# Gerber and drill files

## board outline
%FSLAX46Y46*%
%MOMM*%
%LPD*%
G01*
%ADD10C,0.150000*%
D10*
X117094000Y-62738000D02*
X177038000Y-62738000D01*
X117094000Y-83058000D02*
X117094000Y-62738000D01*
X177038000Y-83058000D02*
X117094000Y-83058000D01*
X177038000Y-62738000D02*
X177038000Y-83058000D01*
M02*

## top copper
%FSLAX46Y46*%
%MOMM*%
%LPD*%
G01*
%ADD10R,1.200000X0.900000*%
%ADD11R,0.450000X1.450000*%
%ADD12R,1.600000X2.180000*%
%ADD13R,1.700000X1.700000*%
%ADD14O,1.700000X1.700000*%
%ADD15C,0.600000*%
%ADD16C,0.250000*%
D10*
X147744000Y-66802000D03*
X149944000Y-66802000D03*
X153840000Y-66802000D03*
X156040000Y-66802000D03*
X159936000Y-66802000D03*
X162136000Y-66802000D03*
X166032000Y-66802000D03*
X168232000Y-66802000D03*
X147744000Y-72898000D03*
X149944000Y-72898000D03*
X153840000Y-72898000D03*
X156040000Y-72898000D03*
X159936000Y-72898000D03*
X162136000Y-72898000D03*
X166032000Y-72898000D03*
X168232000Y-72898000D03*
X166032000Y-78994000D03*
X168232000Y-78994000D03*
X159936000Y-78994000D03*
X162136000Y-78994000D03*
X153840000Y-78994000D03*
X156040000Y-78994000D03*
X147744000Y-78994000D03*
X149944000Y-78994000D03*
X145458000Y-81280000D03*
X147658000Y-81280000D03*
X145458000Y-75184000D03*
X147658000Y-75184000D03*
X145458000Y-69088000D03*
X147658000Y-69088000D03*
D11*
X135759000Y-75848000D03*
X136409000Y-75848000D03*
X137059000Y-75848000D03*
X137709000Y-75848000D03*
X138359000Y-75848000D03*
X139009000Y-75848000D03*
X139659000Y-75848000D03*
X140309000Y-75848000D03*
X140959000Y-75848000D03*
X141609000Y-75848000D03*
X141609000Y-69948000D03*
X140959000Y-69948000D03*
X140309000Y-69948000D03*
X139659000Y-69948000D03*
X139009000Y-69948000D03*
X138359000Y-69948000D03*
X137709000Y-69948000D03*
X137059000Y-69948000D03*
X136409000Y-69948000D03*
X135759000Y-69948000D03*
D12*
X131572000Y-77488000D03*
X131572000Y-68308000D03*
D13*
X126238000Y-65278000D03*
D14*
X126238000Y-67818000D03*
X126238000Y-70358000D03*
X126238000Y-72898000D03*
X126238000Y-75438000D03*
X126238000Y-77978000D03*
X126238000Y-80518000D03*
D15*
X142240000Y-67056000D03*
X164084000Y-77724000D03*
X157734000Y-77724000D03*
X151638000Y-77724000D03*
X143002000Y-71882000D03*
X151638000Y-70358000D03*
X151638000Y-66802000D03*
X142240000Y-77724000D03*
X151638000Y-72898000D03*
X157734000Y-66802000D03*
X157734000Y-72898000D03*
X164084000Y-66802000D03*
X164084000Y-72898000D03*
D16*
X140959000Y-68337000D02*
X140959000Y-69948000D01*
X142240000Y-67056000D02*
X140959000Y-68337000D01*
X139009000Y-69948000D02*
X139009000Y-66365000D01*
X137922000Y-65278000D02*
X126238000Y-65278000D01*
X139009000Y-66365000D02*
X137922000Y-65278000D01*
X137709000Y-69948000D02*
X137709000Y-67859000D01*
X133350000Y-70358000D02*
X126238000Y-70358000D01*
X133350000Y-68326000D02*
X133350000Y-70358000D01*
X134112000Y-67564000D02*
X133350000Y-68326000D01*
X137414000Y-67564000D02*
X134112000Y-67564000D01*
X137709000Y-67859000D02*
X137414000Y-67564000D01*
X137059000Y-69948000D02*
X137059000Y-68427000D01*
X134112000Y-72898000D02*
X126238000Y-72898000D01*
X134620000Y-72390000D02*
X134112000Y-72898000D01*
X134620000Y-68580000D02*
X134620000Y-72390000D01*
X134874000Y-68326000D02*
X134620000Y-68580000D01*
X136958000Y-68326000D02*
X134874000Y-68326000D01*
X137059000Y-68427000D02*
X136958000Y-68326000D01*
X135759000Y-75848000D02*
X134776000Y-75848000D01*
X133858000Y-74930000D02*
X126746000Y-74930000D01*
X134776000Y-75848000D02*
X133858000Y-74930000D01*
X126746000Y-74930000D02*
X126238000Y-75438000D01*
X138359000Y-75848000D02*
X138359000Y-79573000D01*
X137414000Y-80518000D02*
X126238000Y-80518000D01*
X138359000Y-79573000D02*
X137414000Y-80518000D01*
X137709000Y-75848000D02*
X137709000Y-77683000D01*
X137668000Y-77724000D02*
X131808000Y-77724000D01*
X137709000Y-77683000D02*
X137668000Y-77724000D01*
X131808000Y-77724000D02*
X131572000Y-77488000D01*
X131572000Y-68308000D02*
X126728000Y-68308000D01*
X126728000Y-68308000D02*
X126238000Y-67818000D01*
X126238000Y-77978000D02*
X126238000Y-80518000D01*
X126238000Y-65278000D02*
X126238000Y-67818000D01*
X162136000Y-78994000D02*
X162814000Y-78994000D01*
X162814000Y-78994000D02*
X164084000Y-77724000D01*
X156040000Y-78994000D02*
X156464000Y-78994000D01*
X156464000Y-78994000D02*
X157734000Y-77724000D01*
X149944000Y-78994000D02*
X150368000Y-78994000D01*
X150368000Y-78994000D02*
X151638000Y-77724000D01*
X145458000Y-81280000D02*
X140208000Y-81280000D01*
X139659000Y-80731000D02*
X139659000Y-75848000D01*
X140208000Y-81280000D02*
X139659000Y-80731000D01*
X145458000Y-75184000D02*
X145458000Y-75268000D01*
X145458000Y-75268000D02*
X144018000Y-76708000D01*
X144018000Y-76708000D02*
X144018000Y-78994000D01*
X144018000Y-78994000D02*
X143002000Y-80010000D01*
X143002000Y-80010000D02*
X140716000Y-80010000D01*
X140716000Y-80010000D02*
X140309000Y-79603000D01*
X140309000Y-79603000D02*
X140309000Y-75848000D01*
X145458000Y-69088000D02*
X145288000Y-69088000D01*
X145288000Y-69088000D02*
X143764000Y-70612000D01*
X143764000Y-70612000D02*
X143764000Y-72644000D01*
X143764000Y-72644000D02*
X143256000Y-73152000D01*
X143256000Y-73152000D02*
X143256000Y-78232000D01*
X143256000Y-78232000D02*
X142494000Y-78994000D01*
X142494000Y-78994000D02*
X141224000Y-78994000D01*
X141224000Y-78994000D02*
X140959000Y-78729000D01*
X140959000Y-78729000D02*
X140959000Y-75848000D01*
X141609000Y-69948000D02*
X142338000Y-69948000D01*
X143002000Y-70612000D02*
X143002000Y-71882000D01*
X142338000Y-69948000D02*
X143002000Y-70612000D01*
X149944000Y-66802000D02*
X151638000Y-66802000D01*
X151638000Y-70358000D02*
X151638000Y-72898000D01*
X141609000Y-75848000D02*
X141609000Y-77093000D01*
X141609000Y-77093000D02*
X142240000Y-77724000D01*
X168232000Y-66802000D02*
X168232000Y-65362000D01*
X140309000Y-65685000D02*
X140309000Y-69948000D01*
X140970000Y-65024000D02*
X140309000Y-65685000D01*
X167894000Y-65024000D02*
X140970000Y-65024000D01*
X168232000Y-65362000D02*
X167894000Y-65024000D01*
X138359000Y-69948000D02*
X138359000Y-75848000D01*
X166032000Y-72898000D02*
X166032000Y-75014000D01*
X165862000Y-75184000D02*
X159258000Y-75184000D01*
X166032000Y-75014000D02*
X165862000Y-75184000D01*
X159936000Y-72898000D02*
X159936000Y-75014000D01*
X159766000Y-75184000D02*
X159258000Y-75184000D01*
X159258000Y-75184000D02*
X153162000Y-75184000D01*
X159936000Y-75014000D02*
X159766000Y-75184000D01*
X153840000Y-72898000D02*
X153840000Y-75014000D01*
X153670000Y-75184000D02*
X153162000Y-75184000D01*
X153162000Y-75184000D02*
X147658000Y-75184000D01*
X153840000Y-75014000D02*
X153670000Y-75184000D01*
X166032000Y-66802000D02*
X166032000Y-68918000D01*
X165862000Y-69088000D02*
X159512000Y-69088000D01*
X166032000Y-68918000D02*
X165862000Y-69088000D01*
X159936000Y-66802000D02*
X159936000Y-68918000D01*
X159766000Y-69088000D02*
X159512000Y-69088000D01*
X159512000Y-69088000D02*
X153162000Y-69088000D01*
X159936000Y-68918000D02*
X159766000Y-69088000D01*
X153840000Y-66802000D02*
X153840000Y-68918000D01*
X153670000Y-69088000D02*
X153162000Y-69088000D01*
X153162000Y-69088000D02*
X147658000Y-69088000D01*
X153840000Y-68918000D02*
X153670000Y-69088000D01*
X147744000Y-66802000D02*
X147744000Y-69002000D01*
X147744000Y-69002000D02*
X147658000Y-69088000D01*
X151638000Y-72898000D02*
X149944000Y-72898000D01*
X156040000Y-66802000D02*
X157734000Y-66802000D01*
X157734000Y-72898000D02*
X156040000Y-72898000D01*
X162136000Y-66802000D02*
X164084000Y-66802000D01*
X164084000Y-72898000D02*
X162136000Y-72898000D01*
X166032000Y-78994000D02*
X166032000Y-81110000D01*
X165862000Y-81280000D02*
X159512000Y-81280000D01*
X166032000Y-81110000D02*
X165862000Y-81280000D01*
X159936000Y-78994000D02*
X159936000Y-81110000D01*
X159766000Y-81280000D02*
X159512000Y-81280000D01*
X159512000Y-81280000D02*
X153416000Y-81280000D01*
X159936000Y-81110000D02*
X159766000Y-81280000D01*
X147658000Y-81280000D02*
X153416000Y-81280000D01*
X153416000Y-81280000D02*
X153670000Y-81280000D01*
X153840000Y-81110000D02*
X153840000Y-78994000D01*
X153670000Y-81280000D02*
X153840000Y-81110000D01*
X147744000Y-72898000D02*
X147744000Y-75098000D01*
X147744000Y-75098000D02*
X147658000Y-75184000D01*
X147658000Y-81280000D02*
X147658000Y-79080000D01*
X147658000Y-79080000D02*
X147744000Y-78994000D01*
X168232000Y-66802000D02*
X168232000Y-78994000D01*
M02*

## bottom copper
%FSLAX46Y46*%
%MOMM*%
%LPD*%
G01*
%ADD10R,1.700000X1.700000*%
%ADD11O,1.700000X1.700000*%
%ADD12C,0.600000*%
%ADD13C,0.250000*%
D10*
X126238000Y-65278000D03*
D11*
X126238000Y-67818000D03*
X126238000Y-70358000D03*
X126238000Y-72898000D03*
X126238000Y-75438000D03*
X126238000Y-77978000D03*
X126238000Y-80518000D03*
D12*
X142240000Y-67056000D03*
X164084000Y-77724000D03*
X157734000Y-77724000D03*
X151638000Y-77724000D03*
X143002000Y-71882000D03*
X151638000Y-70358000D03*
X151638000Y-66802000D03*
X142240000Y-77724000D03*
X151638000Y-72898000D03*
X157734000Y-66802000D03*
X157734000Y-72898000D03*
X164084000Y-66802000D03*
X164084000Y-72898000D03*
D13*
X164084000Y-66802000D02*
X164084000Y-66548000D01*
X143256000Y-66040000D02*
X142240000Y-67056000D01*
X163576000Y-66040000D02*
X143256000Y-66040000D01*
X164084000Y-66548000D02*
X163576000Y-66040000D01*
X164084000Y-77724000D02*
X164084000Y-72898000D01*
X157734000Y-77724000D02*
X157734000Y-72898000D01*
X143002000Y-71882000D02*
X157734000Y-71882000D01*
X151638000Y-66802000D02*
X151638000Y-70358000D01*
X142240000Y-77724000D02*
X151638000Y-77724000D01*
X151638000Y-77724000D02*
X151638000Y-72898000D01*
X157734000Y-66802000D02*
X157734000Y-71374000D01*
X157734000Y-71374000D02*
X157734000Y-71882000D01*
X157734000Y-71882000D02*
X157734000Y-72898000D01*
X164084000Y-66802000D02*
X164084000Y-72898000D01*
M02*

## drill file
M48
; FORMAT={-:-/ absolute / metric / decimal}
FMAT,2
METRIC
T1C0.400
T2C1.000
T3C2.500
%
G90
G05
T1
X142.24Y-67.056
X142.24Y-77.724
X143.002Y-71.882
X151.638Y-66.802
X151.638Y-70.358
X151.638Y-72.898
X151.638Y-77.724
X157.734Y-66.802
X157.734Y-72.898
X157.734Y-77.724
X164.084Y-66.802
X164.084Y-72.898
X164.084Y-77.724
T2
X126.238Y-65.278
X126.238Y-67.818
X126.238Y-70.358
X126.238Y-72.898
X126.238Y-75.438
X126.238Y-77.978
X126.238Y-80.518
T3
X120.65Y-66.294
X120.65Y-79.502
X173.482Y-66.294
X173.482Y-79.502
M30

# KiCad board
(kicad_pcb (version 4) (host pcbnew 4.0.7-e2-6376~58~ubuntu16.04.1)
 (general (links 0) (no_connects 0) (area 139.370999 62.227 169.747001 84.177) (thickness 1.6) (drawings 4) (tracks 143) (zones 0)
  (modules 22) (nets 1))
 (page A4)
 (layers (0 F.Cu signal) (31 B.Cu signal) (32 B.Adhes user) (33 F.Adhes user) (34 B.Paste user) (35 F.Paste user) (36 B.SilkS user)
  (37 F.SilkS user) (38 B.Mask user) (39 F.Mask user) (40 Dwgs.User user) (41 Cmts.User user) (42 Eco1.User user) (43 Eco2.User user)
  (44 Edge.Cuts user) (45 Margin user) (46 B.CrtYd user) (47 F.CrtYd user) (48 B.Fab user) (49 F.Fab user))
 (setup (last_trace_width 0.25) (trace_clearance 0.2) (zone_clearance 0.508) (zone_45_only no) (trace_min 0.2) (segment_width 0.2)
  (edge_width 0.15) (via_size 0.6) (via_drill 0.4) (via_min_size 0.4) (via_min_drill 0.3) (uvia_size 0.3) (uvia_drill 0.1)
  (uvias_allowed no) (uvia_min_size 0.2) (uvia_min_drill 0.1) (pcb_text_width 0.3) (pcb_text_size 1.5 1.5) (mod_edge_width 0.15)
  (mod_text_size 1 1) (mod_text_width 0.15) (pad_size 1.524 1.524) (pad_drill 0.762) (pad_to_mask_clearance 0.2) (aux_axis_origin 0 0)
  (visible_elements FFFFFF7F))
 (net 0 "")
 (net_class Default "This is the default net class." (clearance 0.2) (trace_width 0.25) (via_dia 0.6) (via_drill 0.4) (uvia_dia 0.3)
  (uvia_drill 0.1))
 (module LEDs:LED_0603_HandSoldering (layer F.Cu) (at 148.844 66.802)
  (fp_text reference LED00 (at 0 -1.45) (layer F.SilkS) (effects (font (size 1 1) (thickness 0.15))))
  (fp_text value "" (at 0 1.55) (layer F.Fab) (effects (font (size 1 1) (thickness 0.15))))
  (pad 1 smd rect (at -1.1 0) (size 1.2 0.9) (layers F.Cu F.Paste F.Mask))
  (pad 2 smd rect (at 1.1 0) (size 1.2 0.9) (layers F.Cu F.Paste F.Mask)))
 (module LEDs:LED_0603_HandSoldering (layer F.Cu) (at 154.94 66.802)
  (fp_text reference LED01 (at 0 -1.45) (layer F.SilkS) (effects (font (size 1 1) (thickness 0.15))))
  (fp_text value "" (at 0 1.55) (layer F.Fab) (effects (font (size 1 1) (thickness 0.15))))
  (pad 1 smd rect (at -1.1 0) (size 1.2 0.9) (layers F.Cu F.Paste F.Mask))
  (pad 2 smd rect (at 1.1 0) (size 1.2 0.9) (layers F.Cu F.Paste F.Mask)))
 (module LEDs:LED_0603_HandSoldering (layer F.Cu) (at 161.036 66.802)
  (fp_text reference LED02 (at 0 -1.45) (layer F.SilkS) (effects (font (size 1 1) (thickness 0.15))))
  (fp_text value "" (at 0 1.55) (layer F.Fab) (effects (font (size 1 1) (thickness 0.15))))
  (pad 1 smd rect (at -1.1 0) (size 1.2 0.9) (layers F.Cu F.Paste F.Mask))
  (pad 2 smd rect (at 1.1 0) (size 1.2 0.9) (layers F.Cu F.Paste F.Mask)))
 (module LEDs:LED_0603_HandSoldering (layer F.Cu) (at 167.132 66.802)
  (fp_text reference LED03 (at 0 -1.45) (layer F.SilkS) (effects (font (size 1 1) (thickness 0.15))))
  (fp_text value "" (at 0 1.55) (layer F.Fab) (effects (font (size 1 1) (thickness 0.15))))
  (pad 1 smd rect (at -1.1 0) (size 1.2 0.9) (layers F.Cu F.Paste F.Mask))
  (pad 2 smd rect (at 1.1 0) (size 1.2 0.9) (layers F.Cu F.Paste F.Mask)))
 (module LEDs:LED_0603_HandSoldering (layer F.Cu) (at 148.844 72.898)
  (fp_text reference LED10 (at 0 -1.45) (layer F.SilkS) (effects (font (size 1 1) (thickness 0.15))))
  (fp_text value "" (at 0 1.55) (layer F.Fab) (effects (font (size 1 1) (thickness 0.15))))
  (pad 1 smd rect (at -1.1 0) (size 1.2 0.9) (layers F.Cu F.Paste F.Mask))
  (pad 2 smd rect (at 1.1 0) (size 1.2 0.9) (layers F.Cu F.Paste F.Mask)))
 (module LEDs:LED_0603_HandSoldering (layer F.Cu) (at 154.94 72.898)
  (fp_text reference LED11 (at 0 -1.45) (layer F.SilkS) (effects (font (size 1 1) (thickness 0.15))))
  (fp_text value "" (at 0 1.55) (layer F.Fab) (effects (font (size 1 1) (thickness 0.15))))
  (pad 1 smd rect (at -1.1 0) (size 1.2 0.9) (layers F.Cu F.Paste F.Mask))
  (pad 2 smd rect (at 1.1 0) (size 1.2 0.9) (layers F.Cu F.Paste F.Mask)))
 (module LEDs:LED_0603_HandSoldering (layer F.Cu) (at 161.036 72.898)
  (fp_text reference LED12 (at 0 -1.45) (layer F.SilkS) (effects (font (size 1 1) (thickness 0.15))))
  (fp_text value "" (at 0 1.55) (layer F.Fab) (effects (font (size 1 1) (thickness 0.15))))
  (pad 1 smd rect (at -1.1 0) (size 1.2 0.9) (layers F.Cu F.Paste F.Mask))
  (pad 2 smd rect (at 1.1 0) (size 1.2 0.9) (layers F.Cu F.Paste F.Mask)))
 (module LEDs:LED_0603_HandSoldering (layer F.Cu) (at 167.132 72.898)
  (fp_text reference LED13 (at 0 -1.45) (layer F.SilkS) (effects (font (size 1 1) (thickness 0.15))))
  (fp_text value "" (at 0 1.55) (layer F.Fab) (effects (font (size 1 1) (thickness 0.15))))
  (pad 1 smd rect (at -1.1 0) (size 1.2 0.9) (layers F.Cu F.Paste F.Mask))
  (pad 2 smd rect (at 1.1 0) (size 1.2 0.9) (layers F.Cu F.Paste F.Mask)))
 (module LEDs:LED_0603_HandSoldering (layer F.Cu) (at 167.132 78.994)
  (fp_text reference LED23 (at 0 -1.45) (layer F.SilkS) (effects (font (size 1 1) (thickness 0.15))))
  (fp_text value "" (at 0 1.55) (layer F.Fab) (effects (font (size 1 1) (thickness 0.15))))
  (pad 1 smd rect (at -1.1 0) (size 1.2 0.9) (layers F.Cu F.Paste F.Mask))
  (pad 2 smd rect (at 1.1 0) (size 1.2 0.9) (layers F.Cu F.Paste F.Mask)))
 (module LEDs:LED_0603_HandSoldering (layer F.Cu) (at 161.036 78.994)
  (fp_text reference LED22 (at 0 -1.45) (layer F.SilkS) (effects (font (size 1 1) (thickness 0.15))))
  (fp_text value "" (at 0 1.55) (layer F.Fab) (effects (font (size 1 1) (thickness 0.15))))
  (pad 1 smd rect (at -1.1 0) (size 1.2 0.9) (layers F.Cu F.Paste F.Mask))
  (pad 2 smd rect (at 1.1 0) (size 1.2 0.9) (layers F.Cu F.Paste F.Mask)))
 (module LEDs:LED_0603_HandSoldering (layer F.Cu) (at 154.94 78.994)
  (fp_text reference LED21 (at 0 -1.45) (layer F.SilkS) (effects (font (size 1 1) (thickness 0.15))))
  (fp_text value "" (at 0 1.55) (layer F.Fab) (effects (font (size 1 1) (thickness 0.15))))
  (pad 1 smd rect (at -1.1 0) (size 1.2 0.9) (layers F.Cu F.Paste F.Mask))
  (pad 2 smd rect (at 1.1 0) (size 1.2 0.9) (layers F.Cu F.Paste F.Mask)))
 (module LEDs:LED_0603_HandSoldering (layer F.Cu) (at 148.844 78.994)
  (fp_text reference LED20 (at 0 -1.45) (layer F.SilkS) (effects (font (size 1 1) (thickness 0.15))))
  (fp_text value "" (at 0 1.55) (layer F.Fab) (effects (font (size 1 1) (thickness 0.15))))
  (pad 1 smd rect (at -1.1 0) (size 1.2 0.9) (layers F.Cu F.Paste F.Mask))
  (pad 2 smd rect (at 1.1 0) (size 1.2 0.9) (layers F.Cu F.Paste F.Mask)))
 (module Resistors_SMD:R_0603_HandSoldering (layer F.Cu) (at 146.558 81.28)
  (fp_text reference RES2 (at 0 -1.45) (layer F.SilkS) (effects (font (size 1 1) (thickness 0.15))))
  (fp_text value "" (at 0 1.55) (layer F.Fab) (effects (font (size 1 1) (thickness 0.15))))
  (pad 1 smd rect (at -1.1 0) (size 1.2 0.9) (layers F.Cu F.Paste F.Mask))
  (pad 2 smd rect (at 1.1 0) (size 1.2 0.9) (layers F.Cu F.Paste F.Mask)))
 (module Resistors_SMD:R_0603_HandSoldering (layer F.Cu) (at 146.558 75.184)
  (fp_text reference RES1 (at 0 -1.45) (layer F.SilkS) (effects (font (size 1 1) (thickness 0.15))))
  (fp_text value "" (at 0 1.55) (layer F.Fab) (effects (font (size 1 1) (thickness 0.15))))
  (pad 1 smd rect (at -1.1 0) (size 1.2 0.9) (layers F.Cu F.Paste F.Mask))
  (pad 2 smd rect (at 1.1 0) (size 1.2 0.9) (layers F.Cu F.Paste F.Mask)))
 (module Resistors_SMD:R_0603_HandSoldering (layer F.Cu) (at 146.558 69.088)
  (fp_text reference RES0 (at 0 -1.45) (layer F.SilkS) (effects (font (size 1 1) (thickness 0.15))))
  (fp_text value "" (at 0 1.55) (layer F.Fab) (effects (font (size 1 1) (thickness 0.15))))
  (pad 1 smd rect (at -1.1 0) (size 1.2 0.9) (layers F.Cu F.Paste F.Mask))
  (pad 2 smd rect (at 1.1 0) (size 1.2 0.9) (layers F.Cu F.Paste F.Mask)))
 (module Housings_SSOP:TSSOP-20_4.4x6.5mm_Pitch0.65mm (layer F.Cu) (at 138.684 72.898 90)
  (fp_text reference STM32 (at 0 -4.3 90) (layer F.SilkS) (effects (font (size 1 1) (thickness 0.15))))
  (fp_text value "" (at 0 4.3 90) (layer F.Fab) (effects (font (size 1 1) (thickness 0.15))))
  (pad 1 smd rect (at -2.95 -2.925 90) (size 1.45 0.45) (layers F.Cu F.Paste F.Mask))
  (pad 2 smd rect (at -2.95 -2.275 90) (size 1.45 0.45) (layers F.Cu F.Paste F.Mask))
  (pad 3 smd rect (at -2.95 -1.625 90) (size 1.45 0.45) (layers F.Cu F.Paste F.Mask))
  (pad 4 smd rect (at -2.95 -0.975 90) (size 1.45 0.45) (layers F.Cu F.Paste F.Mask))
  (pad 5 smd rect (at -2.95 -0.325 90) (size 1.45 0.45) (layers F.Cu F.Paste F.Mask))
  (pad 6 smd rect (at -2.95 0.325 90) (size 1.45 0.45) (layers F.Cu F.Paste F.Mask))
  (pad 7 smd rect (at -2.95 0.975 90) (size 1.45 0.45) (layers F.Cu F.Paste F.Mask))
  (pad 8 smd rect (at -2.95 1.625 90) (size 1.45 0.45) (layers F.Cu F.Paste F.Mask))
  (pad 9 smd rect (at -2.95 2.275 90) (size 1.45 0.45) (layers F.Cu F.Paste F.Mask))
  (pad 10 smd rect (at -2.95 2.925 90) (size 1.45 0.45) (layers F.Cu F.Paste F.Mask))
  (pad 11 smd rect (at 2.95 2.925 90) (size 1.45 0.45) (layers F.Cu F.Paste F.Mask))
  (pad 12 smd rect (at 2.95 2.275 90) (size 1.45 0.45) (layers F.Cu F.Paste F.Mask))
  (pad 13 smd rect (at 2.95 1.625 90) (size 1.45 0.45) (layers F.Cu F.Paste F.Mask))
  (pad 14 smd rect (at 2.95 0.975 90) (size 1.45 0.45) (layers F.Cu F.Paste F.Mask))
  (pad 15 smd rect (at 2.95 0.325 90) (size 1.45 0.45) (layers F.Cu F.Paste F.Mask))
  (pad 16 smd rect (at 2.95 -0.325 90) (size 1.45 0.45) (layers F.Cu F.Paste F.Mask))
  (pad 17 smd rect (at 2.95 -0.975 90) (size 1.45 0.45) (layers F.Cu F.Paste F.Mask))
  (pad 18 smd rect (at 2.95 -1.625 90) (size 1.45 0.45) (layers F.Cu F.Paste F.Mask))
  (pad 19 smd rect (at 2.95 -2.275 90) (size 1.45 0.45) (layers F.Cu F.Paste F.Mask))
  (pad 20 smd rect (at 2.95 -2.925 90) (size 1.45 0.45) (layers F.Cu F.Paste F.Mask)))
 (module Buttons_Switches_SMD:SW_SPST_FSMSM (layer F.Cu) (at 131.572 72.898 90)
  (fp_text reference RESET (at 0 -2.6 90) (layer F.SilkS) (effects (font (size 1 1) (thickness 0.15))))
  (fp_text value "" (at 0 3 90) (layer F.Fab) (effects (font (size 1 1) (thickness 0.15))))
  (pad 1 smd rect (at -4.59 0 90) (size 2.18 1.6) (layers F.Cu F.Paste F.Mask))
  (pad 2 smd rect (at 4.59 0 90) (size 2.18 1.6) (layers F.Cu F.Paste F.Mask)))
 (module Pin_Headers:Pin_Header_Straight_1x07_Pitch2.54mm (layer F.Cu) (at 126.238 65.278)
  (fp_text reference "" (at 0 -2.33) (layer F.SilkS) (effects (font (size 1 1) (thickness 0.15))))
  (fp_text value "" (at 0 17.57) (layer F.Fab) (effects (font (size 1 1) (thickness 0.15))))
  (pad 1 thru_hole rect (at 0 0) (size 1.7 1.7) (drill 1) (layers *.Cu *.Mask))
  (pad 2 thru_hole oval (at 0 2.54) (size 1.7 1.7) (drill 1) (layers *.Cu *.Mask))
  (pad 3 thru_hole oval (at 0 5.08) (size 1.7 1.7) (drill 1) (layers *.Cu *.Mask))
  (pad 4 thru_hole oval (at 0 7.62) (size 1.7 1.7) (drill 1) (layers *.Cu *.Mask))
  (pad 5 thru_hole oval (at 0 10.16) (size 1.7 1.7) (drill 1) (layers *.Cu *.Mask))
  (pad 6 thru_hole oval (at 0 12.7) (size 1.7 1.7) (drill 1) (layers *.Cu *.Mask))
  (pad 7 thru_hole oval (at 0 15.24) (size 1.7 1.7) (drill 1) (layers *.Cu *.Mask)))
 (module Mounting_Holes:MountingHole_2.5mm (layer F.Cu) (at 120.65 66.294)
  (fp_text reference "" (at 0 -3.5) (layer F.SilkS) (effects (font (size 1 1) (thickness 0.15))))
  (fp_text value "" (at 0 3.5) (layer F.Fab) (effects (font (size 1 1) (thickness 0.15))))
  (pad 1 np_thru_hole circle (at 0 0) (size 2.5 2.5) (drill 2.5) (layers *.Cu *.Mask)))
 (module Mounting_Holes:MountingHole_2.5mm (layer F.Cu) (at 120.65 79.502)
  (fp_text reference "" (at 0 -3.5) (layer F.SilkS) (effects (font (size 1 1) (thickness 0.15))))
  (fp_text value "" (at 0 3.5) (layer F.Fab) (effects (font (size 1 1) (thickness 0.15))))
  (pad 1 np_thru_hole circle (at 0 0) (size 2.5 2.5) (drill 2.5) (layers *.Cu *.Mask)))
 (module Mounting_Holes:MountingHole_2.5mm (layer F.Cu) (at 173.482 79.502)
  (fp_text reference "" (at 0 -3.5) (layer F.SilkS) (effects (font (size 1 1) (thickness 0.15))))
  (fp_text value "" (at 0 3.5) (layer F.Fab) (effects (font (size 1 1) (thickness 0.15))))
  (pad 1 np_thru_hole circle (at 0 0) (size 2.5 2.5) (drill 2.5) (layers *.Cu *.Mask)))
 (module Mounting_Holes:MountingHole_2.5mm (layer F.Cu) (at 173.482 66.294)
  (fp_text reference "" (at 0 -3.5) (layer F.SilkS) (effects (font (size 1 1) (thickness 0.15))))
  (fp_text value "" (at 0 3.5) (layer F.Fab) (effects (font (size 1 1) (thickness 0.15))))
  (pad 1 np_thru_hole circle (at 0 0) (size 2.5 2.5) (drill 2.5) (layers *.Cu *.Mask)))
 (gr_line (start 117.094 62.738) (end 177.038 62.738) (angle 90) (layer Edge.Cuts) (width 0.15))
 (gr_line (start 117.094 83.058) (end 117.094 62.738) (angle 90) (layer Edge.Cuts) (width 0.15))
 (gr_line (start 177.038 83.058) (end 117.094 83.058) (angle 90) (layer Edge.Cuts) (width 0.15))
 (gr_line (start 177.038 62.738) (end 177.038 83.058) (angle 90) (layer Edge.Cuts) (width 0.15))
 (segment (start 164.084 66.802) (end 164.084 66.548) (width 0.25) (layer B.Cu) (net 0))
 (segment (start 140.959 68.337) (end 140.959 69.948) (width 0.25) (layer F.Cu) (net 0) (status 800000))
 (segment (start 142.24 67.056) (end 140.959 68.337) (width 0.25) (layer F.Cu) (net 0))
 (via (at 142.24 67.056) (size 0.6) (drill 0.4) (layers F.Cu B.Cu) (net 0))
 (segment (start 143.256 66.04) (end 142.24 67.056) (width 0.25) (layer B.Cu) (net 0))
 (segment (start 163.576 66.04) (end 143.256 66.04) (width 0.25) (layer B.Cu) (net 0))
 (segment (start 164.084 66.548) (end 163.576 66.04) (width 0.25) (layer B.Cu) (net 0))
 (segment (start 139.009 69.948) (end 139.009 66.365) (width 0.25) (layer F.Cu) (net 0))
 (segment (start 137.922 65.278) (end 126.238 65.278) (width 0.25) (layer F.Cu) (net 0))
 (segment (start 139.009 66.365) (end 137.922 65.278) (width 0.25) (layer F.Cu) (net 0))
 (segment (start 137.709 69.948) (end 137.709 67.859) (width 0.25) (layer F.Cu) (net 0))
 (segment (start 133.35 70.358) (end 126.238 70.358) (width 0.25) (layer F.Cu) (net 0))
 (segment (start 133.35 68.326) (end 133.35 70.358) (width 0.25) (layer F.Cu) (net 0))
 (segment (start 134.112 67.564) (end 133.35 68.326) (width 0.25) (layer F.Cu) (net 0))
 (segment (start 137.414 67.564) (end 134.112 67.564) (width 0.25) (layer F.Cu) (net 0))
 (segment (start 137.709 67.859) (end 137.414 67.564) (width 0.25) (layer F.Cu) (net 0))
 (segment (start 137.059 69.948) (end 137.059 68.427) (width 0.25) (layer F.Cu) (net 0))
 (segment (start 134.112 72.898) (end 126.238 72.898) (width 0.25) (layer F.Cu) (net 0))
 (segment (start 134.62 72.39) (end 134.112 72.898) (width 0.25) (layer F.Cu) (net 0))
 (segment (start 134.62 68.58) (end 134.62 72.39) (width 0.25) (layer F.Cu) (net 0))
 (segment (start 134.874 68.326) (end 134.62 68.58) (width 0.25) (layer F.Cu) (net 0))
 (segment (start 136.958 68.326) (end 134.874 68.326) (width 0.25) (layer F.Cu) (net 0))
 (segment (start 137.059 68.427) (end 136.958 68.326) (width 0.25) (layer F.Cu) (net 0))
 (segment (start 135.759 75.848) (end 134.776 75.848) (width 0.25) (layer F.Cu) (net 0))
 (segment (start 133.858 74.93) (end 126.746 74.93) (width 0.25) (layer F.Cu) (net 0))
 (segment (start 134.776 75.848) (end 133.858 74.93) (width 0.25) (layer F.Cu) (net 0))
 (segment (start 126.746 74.93) (end 126.238 75.438) (width 0.25) (layer F.Cu) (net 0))
 (segment (start 138.359 75.848) (end 138.359 79.573) (width 0.25) (layer F.Cu) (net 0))
 (segment (start 137.414 80.518) (end 126.238 80.518) (width 0.25) (layer F.Cu) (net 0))
 (segment (start 138.359 79.573) (end 137.414 80.518) (width 0.25) (layer F.Cu) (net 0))
 (segment (start 137.709 75.848) (end 137.709 77.683) (width 0.25) (layer F.Cu) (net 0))
 (segment (start 137.668 77.724) (end 131.808 77.724) (width 0.25) (layer F.Cu) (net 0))
 (segment (start 137.709 77.683) (end 137.668 77.724) (width 0.25) (layer F.Cu) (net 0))
 (segment (start 131.808 77.724) (end 131.572 77.488) (width 0.25) (layer F.Cu) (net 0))
 (segment (start 131.572 68.308) (end 126.728 68.308) (width 0.25) (layer F.Cu) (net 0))
 (segment (start 126.728 68.308) (end 126.238 67.818) (width 0.25) (layer F.Cu) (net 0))
 (segment (start 126.238 77.978) (end 126.238 80.518) (width 0.25) (layer F.Cu) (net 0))
 (segment (start 126.238 65.278) (end 126.238 67.818) (width 0.25) (layer F.Cu) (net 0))
 (segment (start 162.136 78.994) (end 162.814 78.994) (width 0.25) (layer F.Cu) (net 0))
 (segment (start 164.084 77.724) (end 164.084 72.898) (width 0.25) (layer B.Cu) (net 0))
 (via (at 164.084 77.724) (size 0.6) (drill 0.4) (layers F.Cu B.Cu) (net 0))
 (segment (start 162.814 78.994) (end 164.084 77.724) (width 0.25) (layer F.Cu) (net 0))
 (segment (start 156.04 78.994) (end 156.464 78.994) (width 0.25) (layer F.Cu) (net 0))
 (segment (start 156.464 78.994) (end 157.734 77.724) (width 0.25) (layer F.Cu) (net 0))
 (via (at 157.734 77.724) (size 0.6) (drill 0.4) (layers F.Cu B.Cu) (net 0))
 (segment (start 157.734 77.724) (end 157.734 72.898) (width 0.25) (layer B.Cu) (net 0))
 (segment (start 149.944 78.994) (end 150.368 78.994) (width 0.25) (layer F.Cu) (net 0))
 (segment (start 150.368 78.994) (end 151.638 77.724) (width 0.25) (layer F.Cu) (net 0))
 (via (at 151.638 77.724) (size 0.6) (drill 0.4) (layers F.Cu B.Cu) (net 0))
 (segment (start 145.458 81.28) (end 140.208 81.28) (width 0.25) (layer F.Cu) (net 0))
 (segment (start 139.659 80.731) (end 139.659 75.848) (width 0.25) (layer F.Cu) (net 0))
 (segment (start 140.208 81.28) (end 139.659 80.731) (width 0.25) (layer F.Cu) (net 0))
 (segment (start 145.458 75.184) (end 145.458 75.268) (width 0.25) (layer F.Cu) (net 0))
 (segment (start 145.458 75.268) (end 144.018 76.708) (width 0.25) (layer F.Cu) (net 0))
 (segment (start 144.018 76.708) (end 144.018 78.994) (width 0.25) (layer F.Cu) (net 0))
 (segment (start 144.018 78.994) (end 143.002 80.01) (width 0.25) (layer F.Cu) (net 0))
 (segment (start 143.002 80.01) (end 140.716 80.01) (width 0.25) (layer F.Cu) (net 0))
 (segment (start 140.716 80.01) (end 140.309 79.603) (width 0.25) (layer F.Cu) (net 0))
 (segment (start 140.309 79.603) (end 140.309 75.848) (width 0.25) (layer F.Cu) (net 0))
 (segment (start 145.458 69.088) (end 145.288 69.088) (width 0.25) (layer F.Cu) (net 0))
 (segment (start 145.288 69.088) (end 143.764 70.612) (width 0.25) (layer F.Cu) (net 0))
 (segment (start 143.764 70.612) (end 143.764 72.644) (width 0.25) (layer F.Cu) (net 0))
 (segment (start 143.764 72.644) (end 143.256 73.152) (width 0.25) (layer F.Cu) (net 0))
 (segment (start 143.256 73.152) (end 143.256 78.232) (width 0.25) (layer F.Cu) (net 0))
 (segment (start 143.256 78.232) (end 142.494 78.994) (width 0.25) (layer F.Cu) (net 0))
 (segment (start 142.494 78.994) (end 141.224 78.994) (width 0.25) (layer F.Cu) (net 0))
 (segment (start 141.224 78.994) (end 140.959 78.729) (width 0.25) (layer F.Cu) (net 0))
 (segment (start 140.959 78.729) (end 140.959 75.848) (width 0.25) (layer F.Cu) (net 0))
 (segment (start 141.609 69.948) (end 142.338 69.948) (width 0.25) (layer F.Cu) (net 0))
 (segment (start 143.002 71.882) (end 157.734 71.882) (width 0.25) (layer B.Cu) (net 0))
 (via (at 143.002 71.882) (size 0.6) (drill 0.4) (layers F.Cu B.Cu) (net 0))
 (segment (start 143.002 70.612) (end 143.002 71.882) (width 0.25) (layer F.Cu) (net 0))
 (segment (start 142.338 69.948) (end 143.002 70.612) (width 0.25) (layer F.Cu) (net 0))
 (segment (start 149.944 66.802) (end 151.638 66.802) (width 0.25) (layer F.Cu) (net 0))
 (segment (start 151.638 70.358) (end 151.638 72.898) (width 0.25) (layer F.Cu) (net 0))
 (via (at 151.638 70.358) (size 0.6) (drill 0.4) (layers F.Cu B.Cu) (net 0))
 (segment (start 151.638 66.802) (end 151.638 70.358) (width 0.25) (layer B.Cu) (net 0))
 (via (at 151.638 66.802) (size 0.6) (drill 0.4) (layers F.Cu B.Cu) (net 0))
 (segment (start 141.609 75.848) (end 141.609 77.093) (width 0.25) (layer F.Cu) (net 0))
 (segment (start 142.24 77.724) (end 151.638 77.724) (width 0.25) (layer B.Cu) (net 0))
 (via (at 142.24 77.724) (size 0.6) (drill 0.4) (layers F.Cu B.Cu) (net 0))
 (segment (start 141.609 77.093) (end 142.24 77.724) (width 0.25) (layer F.Cu) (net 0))
 (segment (start 168.232 66.802) (end 168.232 65.362) (width 0.25) (layer F.Cu) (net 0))
 (segment (start 140.309 65.685) (end 140.309 69.948) (width 0.25) (layer F.Cu) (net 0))
 (segment (start 140.97 65.024) (end 140.309 65.685) (width 0.25) (layer F.Cu) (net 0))
 (segment (start 167.894 65.024) (end 140.97 65.024) (width 0.25) (layer F.Cu) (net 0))
 (segment (start 168.232 65.362) (end 167.894 65.024) (width 0.25) (layer F.Cu) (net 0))
 (segment (start 138.359 69.948) (end 138.359 75.848) (width 0.25) (layer F.Cu) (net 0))
 (segment (start 166.032 72.898) (end 166.032 75.014) (width 0.25) (layer F.Cu) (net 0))
 (segment (start 165.862 75.184) (end 159.258 75.184) (width 0.25) (layer F.Cu) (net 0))
 (segment (start 166.032 75.014) (end 165.862 75.184) (width 0.25) (layer F.Cu) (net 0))
 (segment (start 159.936 72.898) (end 159.936 75.014) (width 0.25) (layer F.Cu) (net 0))
 (segment (start 159.766 75.184) (end 159.258 75.184) (width 0.25) (layer F.Cu) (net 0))
 (segment (start 159.258 75.184) (end 153.162 75.184) (width 0.25) (layer F.Cu) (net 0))
 (segment (start 159.936 75.014) (end 159.766 75.184) (width 0.25) (layer F.Cu) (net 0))
 (segment (start 153.84 72.898) (end 153.84 75.014) (width 0.25) (layer F.Cu) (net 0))
 (segment (start 153.67 75.184) (end 153.162 75.184) (width 0.25) (layer F.Cu) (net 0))
 (segment (start 153.162 75.184) (end 147.658 75.184) (width 0.25) (layer F.Cu) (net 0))
 (segment (start 153.84 75.014) (end 153.67 75.184) (width 0.25) (layer F.Cu) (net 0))
 (segment (start 166.032 66.802) (end 166.032 68.918) (width 0.25) (layer F.Cu) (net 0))
 (segment (start 165.862 69.088) (end 159.512 69.088) (width 0.25) (layer F.Cu) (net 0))
 (segment (start 166.032 68.918) (end 165.862 69.088) (width 0.25) (layer F.Cu) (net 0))
 (segment (start 159.936 66.802) (end 159.936 68.918) (width 0.25) (layer F.Cu) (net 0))
 (segment (start 159.766 69.088) (end 159.512 69.088) (width 0.25) (layer F.Cu) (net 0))
 (segment (start 159.512 69.088) (end 153.162 69.088) (width 0.25) (layer F.Cu) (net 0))
 (segment (start 159.936 68.918) (end 159.766 69.088) (width 0.25) (layer F.Cu) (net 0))
 (segment (start 153.84 66.802) (end 153.84 68.918) (width 0.25) (layer F.Cu) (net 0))
 (segment (start 153.67 69.088) (end 153.162 69.088) (width 0.25) (layer F.Cu) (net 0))
 (segment (start 153.162 69.088) (end 147.658 69.088) (width 0.25) (layer F.Cu) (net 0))
 (segment (start 153.84 68.918) (end 153.67 69.088) (width 0.25) (layer F.Cu) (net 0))
 (segment (start 147.744 66.802) (end 147.744 69.002) (width 0.25) (layer F.Cu) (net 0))
 (segment (start 147.744 69.002) (end 147.658 69.088) (width 0.25) (layer F.Cu) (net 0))
 (segment (start 151.638 77.724) (end 151.638 72.898) (width 0.25) (layer B.Cu) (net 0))
 (segment (start 151.638 72.898) (end 149.944 72.898) (width 0.25) (layer F.Cu) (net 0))
 (via (at 151.638 72.898) (size 0.6) (drill 0.4) (layers F.Cu B.Cu) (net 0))
 (segment (start 156.04 66.802) (end 157.734 66.802) (width 0.25) (layer F.Cu) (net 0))
 (via (at 157.734 66.802) (size 0.6) (drill 0.4) (layers F.Cu B.Cu) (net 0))
 (segment (start 157.734 66.802) (end 157.734 71.374) (width 0.25) (layer B.Cu) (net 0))
 (segment (start 157.734 71.374) (end 157.734 71.882) (width 0.25) (layer B.Cu) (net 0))
 (segment (start 157.734 71.882) (end 157.734 72.898) (width 0.25) (layer B.Cu) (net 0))
 (segment (start 157.734 72.898) (end 156.04 72.898) (width 0.25) (layer F.Cu) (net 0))
 (via (at 157.734 72.898) (size 0.6) (drill 0.4) (layers F.Cu B.Cu) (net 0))
 (segment (start 162.136 66.802) (end 164.084 66.802) (width 0.25) (layer F.Cu) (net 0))
 (via (at 164.084 66.802) (size 0.6) (drill 0.4) (layers F.Cu B.Cu) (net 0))
 (segment (start 164.084 66.802) (end 164.084 72.898) (width 0.25) (layer B.Cu) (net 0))
 (segment (start 164.084 72.898) (end 162.136 72.898) (width 0.25) (layer F.Cu) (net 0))
 (via (at 164.084 72.898) (size 0.6) (drill 0.4) (layers F.Cu B.Cu) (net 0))
 (segment (start 166.032 78.994) (end 166.032 81.11) (width 0.25) (layer F.Cu) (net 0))
 (segment (start 165.862 81.28) (end 159.512 81.28) (width 0.25) (layer F.Cu) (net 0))
 (segment (start 166.032 81.11) (end 165.862 81.28) (width 0.25) (layer F.Cu) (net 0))
 (segment (start 159.936 78.994) (end 159.936 81.11) (width 0.25) (layer F.Cu) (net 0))
 (segment (start 159.766 81.28) (end 159.512 81.28) (width 0.25) (layer F.Cu) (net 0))
 (segment (start 159.512 81.28) (end 153.416 81.28) (width 0.25) (layer F.Cu) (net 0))
 (segment (start 159.936 81.11) (end 159.766 81.28) (width 0.25) (layer F.Cu) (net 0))
 (segment (start 147.658 81.28) (end 153.416 81.28) (width 0.25) (layer F.Cu) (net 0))
 (segment (start 153.416 81.28) (end 153.67 81.28) (width 0.25) (layer F.Cu) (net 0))
 (segment (start 153.84 81.11) (end 153.84 78.994) (width 0.25) (layer F.Cu) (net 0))
 (segment (start 153.67 81.28) (end 153.84 81.11) (width 0.25) (layer F.Cu) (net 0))
 (segment (start 147.744 72.898) (end 147.744 75.098) (width 0.25) (layer F.Cu) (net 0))
 (segment (start 147.744 75.098) (end 147.658 75.184) (width 0.25) (layer F.Cu) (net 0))
 (segment (start 147.658 81.28) (end 147.658 79.08) (width 0.25) (layer F.Cu) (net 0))
 (segment (start 147.658 79.08) (end 147.744 78.994) (width 0.25) (layer F.Cu) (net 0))
 (segment (start 168.232 66.802) (end 168.232 78.994) (width 0.25) (layer F.Cu) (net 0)))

